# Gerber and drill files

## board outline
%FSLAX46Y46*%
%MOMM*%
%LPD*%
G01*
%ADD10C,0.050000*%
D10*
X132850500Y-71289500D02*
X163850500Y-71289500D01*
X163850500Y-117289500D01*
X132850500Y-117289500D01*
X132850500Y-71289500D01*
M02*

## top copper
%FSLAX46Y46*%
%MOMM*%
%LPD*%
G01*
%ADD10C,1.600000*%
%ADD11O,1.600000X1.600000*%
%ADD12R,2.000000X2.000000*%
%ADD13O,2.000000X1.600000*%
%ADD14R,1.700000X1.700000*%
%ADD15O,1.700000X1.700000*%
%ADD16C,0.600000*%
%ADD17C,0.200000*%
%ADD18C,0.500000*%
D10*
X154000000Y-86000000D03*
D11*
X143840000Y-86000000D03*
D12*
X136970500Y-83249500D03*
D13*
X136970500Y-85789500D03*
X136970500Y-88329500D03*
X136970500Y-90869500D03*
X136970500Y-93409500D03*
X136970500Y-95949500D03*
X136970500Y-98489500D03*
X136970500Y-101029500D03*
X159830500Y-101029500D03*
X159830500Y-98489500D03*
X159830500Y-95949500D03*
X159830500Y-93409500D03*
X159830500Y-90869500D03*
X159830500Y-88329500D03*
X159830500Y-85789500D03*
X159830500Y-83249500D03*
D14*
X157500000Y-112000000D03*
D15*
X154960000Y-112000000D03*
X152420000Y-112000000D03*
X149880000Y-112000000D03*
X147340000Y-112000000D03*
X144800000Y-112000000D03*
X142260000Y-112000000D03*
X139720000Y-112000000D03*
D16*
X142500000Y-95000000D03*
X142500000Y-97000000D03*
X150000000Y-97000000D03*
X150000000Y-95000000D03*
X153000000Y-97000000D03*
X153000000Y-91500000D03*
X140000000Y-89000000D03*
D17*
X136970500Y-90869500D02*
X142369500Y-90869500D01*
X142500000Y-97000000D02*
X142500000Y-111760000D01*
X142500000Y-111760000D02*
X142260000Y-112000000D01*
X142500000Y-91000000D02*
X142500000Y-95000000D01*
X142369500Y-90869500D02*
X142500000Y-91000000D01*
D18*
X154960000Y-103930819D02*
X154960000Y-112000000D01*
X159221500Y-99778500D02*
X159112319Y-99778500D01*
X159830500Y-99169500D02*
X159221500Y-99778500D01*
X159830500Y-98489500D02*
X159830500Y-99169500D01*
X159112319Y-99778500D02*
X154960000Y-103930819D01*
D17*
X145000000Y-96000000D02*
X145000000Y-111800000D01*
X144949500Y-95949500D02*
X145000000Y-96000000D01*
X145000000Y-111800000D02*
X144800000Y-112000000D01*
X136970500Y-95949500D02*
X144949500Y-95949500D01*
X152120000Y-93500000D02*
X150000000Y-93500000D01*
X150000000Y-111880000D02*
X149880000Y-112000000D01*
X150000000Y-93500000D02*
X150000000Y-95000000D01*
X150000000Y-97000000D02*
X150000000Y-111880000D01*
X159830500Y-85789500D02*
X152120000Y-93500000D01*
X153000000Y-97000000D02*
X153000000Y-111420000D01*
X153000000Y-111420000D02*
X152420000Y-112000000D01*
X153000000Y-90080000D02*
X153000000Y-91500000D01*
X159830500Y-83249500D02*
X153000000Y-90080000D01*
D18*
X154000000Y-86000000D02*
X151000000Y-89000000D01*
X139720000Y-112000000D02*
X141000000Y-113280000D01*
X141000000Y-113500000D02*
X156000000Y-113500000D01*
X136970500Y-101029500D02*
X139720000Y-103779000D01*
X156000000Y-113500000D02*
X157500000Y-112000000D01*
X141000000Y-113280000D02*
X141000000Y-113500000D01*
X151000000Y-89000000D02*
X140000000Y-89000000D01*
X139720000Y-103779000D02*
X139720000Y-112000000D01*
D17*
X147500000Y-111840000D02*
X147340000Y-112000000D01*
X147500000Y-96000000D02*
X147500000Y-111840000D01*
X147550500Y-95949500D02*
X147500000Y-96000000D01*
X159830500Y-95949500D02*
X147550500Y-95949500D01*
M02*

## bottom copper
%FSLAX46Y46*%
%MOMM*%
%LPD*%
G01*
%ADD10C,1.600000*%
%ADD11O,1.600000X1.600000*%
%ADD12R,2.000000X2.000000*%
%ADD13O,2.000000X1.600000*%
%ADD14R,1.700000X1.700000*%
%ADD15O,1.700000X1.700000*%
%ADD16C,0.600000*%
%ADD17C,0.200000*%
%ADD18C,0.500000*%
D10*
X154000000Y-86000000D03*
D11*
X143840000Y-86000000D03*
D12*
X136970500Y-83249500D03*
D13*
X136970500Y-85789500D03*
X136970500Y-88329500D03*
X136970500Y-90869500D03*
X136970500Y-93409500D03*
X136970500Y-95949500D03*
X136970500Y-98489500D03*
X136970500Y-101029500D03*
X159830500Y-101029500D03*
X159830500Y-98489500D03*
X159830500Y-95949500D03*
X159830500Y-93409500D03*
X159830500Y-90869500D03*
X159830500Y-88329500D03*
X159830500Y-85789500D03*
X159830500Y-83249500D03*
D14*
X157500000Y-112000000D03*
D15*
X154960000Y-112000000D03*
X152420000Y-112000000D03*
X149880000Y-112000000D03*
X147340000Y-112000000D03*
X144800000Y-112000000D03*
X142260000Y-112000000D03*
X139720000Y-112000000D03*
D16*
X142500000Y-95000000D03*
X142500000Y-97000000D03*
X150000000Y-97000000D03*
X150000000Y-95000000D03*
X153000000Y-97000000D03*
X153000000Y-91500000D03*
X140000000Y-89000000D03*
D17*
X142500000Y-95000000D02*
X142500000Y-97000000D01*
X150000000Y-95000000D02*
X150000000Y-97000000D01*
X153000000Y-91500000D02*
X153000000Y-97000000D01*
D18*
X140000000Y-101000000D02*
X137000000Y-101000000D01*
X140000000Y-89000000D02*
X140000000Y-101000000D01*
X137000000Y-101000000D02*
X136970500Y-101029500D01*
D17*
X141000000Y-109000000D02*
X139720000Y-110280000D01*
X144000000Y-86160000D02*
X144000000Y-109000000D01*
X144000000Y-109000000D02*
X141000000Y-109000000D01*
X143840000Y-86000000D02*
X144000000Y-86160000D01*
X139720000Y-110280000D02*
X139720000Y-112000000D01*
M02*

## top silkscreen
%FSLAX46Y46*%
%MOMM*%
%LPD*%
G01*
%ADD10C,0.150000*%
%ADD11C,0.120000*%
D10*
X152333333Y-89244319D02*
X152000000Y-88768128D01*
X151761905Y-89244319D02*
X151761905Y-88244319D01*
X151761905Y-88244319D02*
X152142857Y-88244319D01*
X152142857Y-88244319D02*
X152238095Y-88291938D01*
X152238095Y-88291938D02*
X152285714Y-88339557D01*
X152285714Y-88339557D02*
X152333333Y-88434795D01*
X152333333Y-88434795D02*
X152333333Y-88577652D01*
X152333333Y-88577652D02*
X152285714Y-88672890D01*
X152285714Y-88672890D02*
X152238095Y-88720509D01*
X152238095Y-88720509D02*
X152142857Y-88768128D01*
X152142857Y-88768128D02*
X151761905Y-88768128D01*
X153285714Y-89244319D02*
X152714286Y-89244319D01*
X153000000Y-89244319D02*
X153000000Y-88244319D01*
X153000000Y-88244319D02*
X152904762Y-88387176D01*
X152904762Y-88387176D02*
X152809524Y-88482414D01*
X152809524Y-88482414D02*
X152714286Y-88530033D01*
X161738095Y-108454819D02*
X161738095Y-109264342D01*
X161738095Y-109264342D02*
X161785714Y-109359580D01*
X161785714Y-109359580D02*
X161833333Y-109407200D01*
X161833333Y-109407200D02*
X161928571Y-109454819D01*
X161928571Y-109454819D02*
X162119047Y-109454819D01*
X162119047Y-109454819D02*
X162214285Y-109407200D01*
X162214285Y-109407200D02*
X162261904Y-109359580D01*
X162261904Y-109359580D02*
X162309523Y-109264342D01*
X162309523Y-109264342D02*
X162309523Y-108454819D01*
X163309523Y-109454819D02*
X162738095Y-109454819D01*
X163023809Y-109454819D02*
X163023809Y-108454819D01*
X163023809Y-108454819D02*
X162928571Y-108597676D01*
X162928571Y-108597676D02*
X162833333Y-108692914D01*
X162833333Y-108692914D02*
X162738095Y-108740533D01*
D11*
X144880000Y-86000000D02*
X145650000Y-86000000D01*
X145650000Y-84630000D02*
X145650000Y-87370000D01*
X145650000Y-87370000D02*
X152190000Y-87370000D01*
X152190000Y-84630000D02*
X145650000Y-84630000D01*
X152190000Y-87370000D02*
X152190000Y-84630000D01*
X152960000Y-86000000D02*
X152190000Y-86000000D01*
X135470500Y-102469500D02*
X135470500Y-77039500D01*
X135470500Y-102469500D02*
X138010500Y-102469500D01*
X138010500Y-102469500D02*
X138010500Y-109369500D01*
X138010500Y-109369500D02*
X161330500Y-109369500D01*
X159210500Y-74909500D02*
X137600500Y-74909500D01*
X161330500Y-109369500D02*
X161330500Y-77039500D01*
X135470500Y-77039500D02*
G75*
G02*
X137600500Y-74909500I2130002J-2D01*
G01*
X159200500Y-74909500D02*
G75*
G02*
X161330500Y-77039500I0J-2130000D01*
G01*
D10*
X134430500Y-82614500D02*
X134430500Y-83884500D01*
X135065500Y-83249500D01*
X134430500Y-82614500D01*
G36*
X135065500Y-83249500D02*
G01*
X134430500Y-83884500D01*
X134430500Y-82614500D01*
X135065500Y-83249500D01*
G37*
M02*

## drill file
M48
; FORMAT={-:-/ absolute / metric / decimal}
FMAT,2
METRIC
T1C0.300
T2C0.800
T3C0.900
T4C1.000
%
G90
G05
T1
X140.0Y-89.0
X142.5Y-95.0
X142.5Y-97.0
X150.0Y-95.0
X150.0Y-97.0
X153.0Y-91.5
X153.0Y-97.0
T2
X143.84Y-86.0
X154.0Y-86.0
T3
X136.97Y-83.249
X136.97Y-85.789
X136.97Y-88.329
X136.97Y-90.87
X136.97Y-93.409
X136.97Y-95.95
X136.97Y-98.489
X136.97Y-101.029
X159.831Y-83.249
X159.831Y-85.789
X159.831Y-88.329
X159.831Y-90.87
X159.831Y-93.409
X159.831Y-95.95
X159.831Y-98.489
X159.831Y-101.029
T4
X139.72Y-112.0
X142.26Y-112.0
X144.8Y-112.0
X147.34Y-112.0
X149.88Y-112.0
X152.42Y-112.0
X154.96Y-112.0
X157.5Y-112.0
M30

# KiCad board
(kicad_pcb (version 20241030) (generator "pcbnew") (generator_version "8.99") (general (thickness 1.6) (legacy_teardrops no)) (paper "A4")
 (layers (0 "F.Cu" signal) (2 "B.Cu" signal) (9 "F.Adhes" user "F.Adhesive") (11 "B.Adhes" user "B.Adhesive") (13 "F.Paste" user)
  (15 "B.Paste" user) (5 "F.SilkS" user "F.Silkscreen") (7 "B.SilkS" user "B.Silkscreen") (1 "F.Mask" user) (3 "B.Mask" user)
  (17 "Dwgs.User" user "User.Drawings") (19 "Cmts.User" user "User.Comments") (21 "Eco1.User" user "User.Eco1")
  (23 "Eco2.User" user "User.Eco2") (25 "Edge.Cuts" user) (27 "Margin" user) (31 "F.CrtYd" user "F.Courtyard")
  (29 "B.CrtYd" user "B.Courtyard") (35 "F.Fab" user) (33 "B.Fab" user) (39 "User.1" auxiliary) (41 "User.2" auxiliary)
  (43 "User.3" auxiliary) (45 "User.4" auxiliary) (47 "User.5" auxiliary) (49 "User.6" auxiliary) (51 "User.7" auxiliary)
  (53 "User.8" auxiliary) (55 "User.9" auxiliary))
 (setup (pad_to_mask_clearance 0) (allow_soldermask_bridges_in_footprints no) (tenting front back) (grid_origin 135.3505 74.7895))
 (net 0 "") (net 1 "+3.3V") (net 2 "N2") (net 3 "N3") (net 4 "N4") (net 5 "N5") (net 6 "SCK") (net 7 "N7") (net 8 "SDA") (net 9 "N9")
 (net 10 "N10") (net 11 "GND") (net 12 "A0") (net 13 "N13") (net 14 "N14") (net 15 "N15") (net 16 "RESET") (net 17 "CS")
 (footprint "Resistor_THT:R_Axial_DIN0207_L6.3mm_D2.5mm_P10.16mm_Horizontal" (layer "F.Cu") (at 154 86 180)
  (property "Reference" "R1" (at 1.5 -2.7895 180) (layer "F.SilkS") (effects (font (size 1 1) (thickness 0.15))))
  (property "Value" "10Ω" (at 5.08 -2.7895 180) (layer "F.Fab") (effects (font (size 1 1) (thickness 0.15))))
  (fp_line (start 9.12 0) (end 8.35 0) (stroke (width 0.12) (type solid)) (layer "F.SilkS"))
  (fp_line (start 8.35 1.37) (end 8.35 -1.37) (stroke (width 0.12) (type solid)) (layer "F.SilkS"))
  (fp_line (start 8.35 -1.37) (end 1.81 -1.37) (stroke (width 0.12) (type solid)) (layer "F.SilkS"))
  (fp_line (start 1.81 1.37) (end 8.35 1.37) (stroke (width 0.12) (type solid)) (layer "F.SilkS"))
  (fp_line (start 1.81 -1.37) (end 1.81 1.37) (stroke (width 0.12) (type solid)) (layer "F.SilkS"))
  (fp_line (start 1.04 0) (end 1.81 0) (stroke (width 0.12) (type solid)) (layer "F.SilkS"))
  (pad "1" thru_hole circle (at 0 0 180) (size 1.6 1.6) (drill 0.8) (layers "F&B.Cu" "*.Mask") (remove_unused_layers no) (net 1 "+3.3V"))
  (pad "2" thru_hole oval (at 10.16 0 180) (size 1.6 1.6) (drill 0.8) (layers "F&B.Cu" "*.Mask") (remove_unused_layers no) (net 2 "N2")))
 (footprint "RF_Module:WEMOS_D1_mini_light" (layer "F.Cu") (at 136.9705 83.2495)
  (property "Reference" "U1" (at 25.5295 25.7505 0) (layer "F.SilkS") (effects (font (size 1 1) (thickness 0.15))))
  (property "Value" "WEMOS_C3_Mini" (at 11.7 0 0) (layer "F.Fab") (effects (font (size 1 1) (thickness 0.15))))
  (fp_line (start -1.5 19.22) (end -1.5 -6.21) (stroke (width 0.12) (type solid)) (layer "F.SilkS"))
  (fp_line (start -1.5 19.22) (end 1.04 19.22) (stroke (width 0.12) (type solid)) (layer "F.SilkS"))
  (fp_line (start 1.04 19.22) (end 1.04 26.12) (stroke (width 0.12) (type solid)) (layer "F.SilkS"))
  (fp_line (start 1.04 26.12) (end 24.36 26.12) (stroke (width 0.12) (type solid)) (layer "F.SilkS"))
  (fp_line (start 22.24 -8.34) (end 0.63 -8.34) (stroke (width 0.12) (type solid)) (layer "F.SilkS"))
  (fp_line (start 24.36 26.12) (end 24.36 -6.21) (stroke (width 0.12) (type solid)) (layer "F.SilkS"))
  (fp_arc (start -1.5 -6.21) (mid -0.876137 -7.716137) (end 0.63 -8.34) (stroke (width 0.12) (type solid)) (layer "F.SilkS"))
  (fp_arc (start 22.23 -8.34) (mid 23.736137 -7.716137) (end 24.36 -6.21) (stroke (width 0.12) (type solid)) (layer "F.SilkS"))
  (fp_poly (pts (xy -2.54 -0.635) (xy -2.54 0.635) (xy -1.905 0)) (stroke (width 0.15) (type solid)) (fill solid) (layer "F.SilkS"))
  (pad "1" thru_hole rect (at 0 0) (size 2 2) (drill 0.9) (layers "*.Cu" "*.Mask") (remove_unused_layers no) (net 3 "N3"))
  (pad "2" thru_hole oval (at 0 2.54) (size 2 1.6) (drill 0.9) (layers "*.Cu" "*.Mask") (remove_unused_layers no) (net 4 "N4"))
  (pad "3" thru_hole oval (at 0 5.08) (size 2 1.6) (drill 0.9) (layers "*.Cu" "*.Mask") (remove_unused_layers no) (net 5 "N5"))
  (pad "4" thru_hole oval (at 0 7.62) (size 2 1.6) (drill 0.9) (layers "*.Cu" "*.Mask") (remove_unused_layers no) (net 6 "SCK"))
  (pad "5" thru_hole oval (at 0 10.16) (size 2 1.6) (drill 0.9) (layers "*.Cu" "*.Mask") (remove_unused_layers no) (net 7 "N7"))
  (pad "6" thru_hole oval (at 0 12.7) (size 2 1.6) (drill 0.9) (layers "*.Cu" "*.Mask") (remove_unused_layers no) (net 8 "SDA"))
  (pad "7" thru_hole oval (at 0 15.24) (size 2 1.6) (drill 0.9) (layers "*.Cu" "*.Mask") (remove_unused_layers no) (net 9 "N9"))
  (pad "8" thru_hole oval (at 0 17.78) (size 2 1.6) (drill 0.9) (layers "*.Cu" "*.Mask") (remove_unused_layers no) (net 1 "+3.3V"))
  (pad "9" thru_hole oval (at 22.86 17.78) (size 2 1.6) (drill 0.9) (layers "*.Cu" "*.Mask") (remove_unused_layers no) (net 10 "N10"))
  (pad "10" thru_hole oval (at 22.86 15.24) (size 2 1.6) (drill 0.9) (layers "*.Cu" "*.Mask") (remove_unused_layers no) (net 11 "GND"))
  (pad "11" thru_hole oval (at 22.86 12.7) (size 2 1.6) (drill 0.9) (layers "*.Cu" "*.Mask") (remove_unused_layers no) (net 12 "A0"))
  (pad "12" thru_hole oval (at 22.86 10.16) (size 2 1.6) (drill 0.9) (layers "*.Cu" "*.Mask") (remove_unused_layers no) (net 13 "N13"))
  (pad "13" thru_hole oval (at 22.86 7.62) (size 2 1.6) (drill 0.9) (layers "*.Cu" "*.Mask") (remove_unused_layers no) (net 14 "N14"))
  (pad "14" thru_hole oval (at 22.86 5.08) (size 2 1.6) (drill 0.9) (layers "*.Cu" "*.Mask") (remove_unused_layers no) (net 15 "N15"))
  (pad "15" thru_hole oval (at 22.86 2.54) (size 2 1.6) (drill 0.9) (layers "*.Cu" "*.Mask") (remove_unused_layers no) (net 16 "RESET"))
  (pad "16" thru_hole oval (at 22.86 0) (size 2 1.6) (drill 0.9) (layers "*.Cu" "*.Mask") (remove_unused_layers no) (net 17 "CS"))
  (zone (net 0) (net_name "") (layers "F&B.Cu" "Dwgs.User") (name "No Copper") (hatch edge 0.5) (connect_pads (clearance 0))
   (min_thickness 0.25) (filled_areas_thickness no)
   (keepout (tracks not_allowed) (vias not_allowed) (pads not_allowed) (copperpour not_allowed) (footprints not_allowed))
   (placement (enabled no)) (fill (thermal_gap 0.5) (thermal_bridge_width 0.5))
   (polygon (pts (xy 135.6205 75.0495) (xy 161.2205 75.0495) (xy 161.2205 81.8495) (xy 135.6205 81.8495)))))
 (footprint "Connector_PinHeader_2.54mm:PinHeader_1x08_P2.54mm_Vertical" (layer "B.Cu") (at 157.5 112 90)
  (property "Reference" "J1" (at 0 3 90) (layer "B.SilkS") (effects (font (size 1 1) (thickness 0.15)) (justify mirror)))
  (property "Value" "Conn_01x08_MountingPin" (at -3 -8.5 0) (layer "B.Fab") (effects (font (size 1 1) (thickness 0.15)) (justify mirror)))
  (pad "1" thru_hole rect (at 0 0 90) (size 1.7 1.7) (drill 1) (layers "F&B.Cu" "*.Mask") (remove_unused_layers no) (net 1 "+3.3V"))
  (pad "2" thru_hole oval (at 0 -2.54 90) (size 1.7 1.7) (drill 1) (layers "F&B.Cu" "*.Mask") (remove_unused_layers no) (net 11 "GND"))
  (pad "3" thru_hole oval (at 0 -5.08 90) (size 1.7 1.7) (drill 1) (layers "F&B.Cu" "*.Mask") (remove_unused_layers no) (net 17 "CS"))
  (pad "4" thru_hole oval (at 0 -7.62 90) (size 1.7 1.7) (drill 1) (layers "F&B.Cu" "*.Mask") (remove_unused_layers no) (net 16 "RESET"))
  (pad "5" thru_hole oval (at 0 -10.16 90) (size 1.7 1.7) (drill 1) (layers "F&B.Cu" "*.Mask") (remove_unused_layers no) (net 12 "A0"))
  (pad "6" thru_hole oval (at 0 -12.7 90) (size 1.7 1.7) (drill 1) (layers "F&B.Cu" "*.Mask") (remove_unused_layers no) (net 8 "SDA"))
  (pad "7" thru_hole oval (at 0 -15.24 90) (size 1.7 1.7) (drill 1) (layers "F&B.Cu" "*.Mask") (remove_unused_layers no) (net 6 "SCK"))
  (pad "8" thru_hole oval (at 0 -17.78 90) (size 1.7 1.7) (drill 1) (layers "F&B.Cu" "*.Mask") (remove_unused_layers no) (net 2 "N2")))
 (gr_rect (start 132.8505 71.2895) (end 163.8505 117.2895) (stroke (width 0.05) (type default)) (fill none) (layer "Edge.Cuts"))
 (segment (start 136.9705 90.8695) (end 142.3695 90.8695) (width 0.2) (layer "F.Cu") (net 6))
 (segment (start 142.5 97) (end 142.5 111.76) (width 0.2) (layer "F.Cu") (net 6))
 (segment (start 142.5 111.76) (end 142.26 112) (width 0.2) (layer "F.Cu") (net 6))
 (segment (start 142.5 91) (end 142.5 95) (width 0.2) (layer "F.Cu") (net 6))
 (segment (start 142.3695 90.8695) (end 142.5 91) (width 0.2) (layer "F.Cu") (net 6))
 (via (at 142.5 95) (size 0.6) (drill 0.3) (layers "F.Cu" "B.Cu") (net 6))
 (via (at 142.5 97) (size 0.6) (drill 0.3) (layers "F.Cu" "B.Cu") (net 6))
 (segment (start 142.5 95) (end 142.5 97) (width 0.2) (layer "B.Cu") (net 6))
 (segment (start 154.96 103.930819) (end 154.96 112) (width 0.5) (layer "F.Cu") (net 11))
 (segment (start 159.2215 99.7785) (end 159.112319 99.7785) (width 0.5) (layer "F.Cu") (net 11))
 (segment (start 159.8305 99.1695) (end 159.2215 99.7785) (width 0.5) (layer "F.Cu") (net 11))
 (segment (start 159.8305 98.4895) (end 159.8305 99.1695) (width 0.5) (layer "F.Cu") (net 11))
 (segment (start 159.112319 99.7785) (end 154.96 103.930819) (width 0.5) (layer "F.Cu") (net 11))
 (segment (start 145 96) (end 145 111.8) (width 0.2) (layer "F.Cu") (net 8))
 (segment (start 144.9495 95.9495) (end 145 96) (width 0.2) (layer "F.Cu") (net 8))
 (segment (start 145 111.8) (end 144.8 112) (width 0.2) (layer "F.Cu") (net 8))
 (segment (start 136.9705 95.9495) (end 144.9495 95.9495) (width 0.2) (layer "F.Cu") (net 8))
 (segment (start 152.12 93.5) (end 150 93.5) (width 0.2) (layer "F.Cu") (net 16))
 (segment (start 150 111.88) (end 149.88 112) (width 0.2) (layer "F.Cu") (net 16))
 (segment (start 150 93.5) (end 150 95) (width 0.2) (layer "F.Cu") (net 16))
 (segment (start 150 97) (end 150 111.88) (width 0.2) (layer "F.Cu") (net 16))
 (segment (start 159.8305 85.7895) (end 152.12 93.5) (width 0.2) (layer "F.Cu") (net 16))
 (via (at 150 97) (size 0.6) (drill 0.3) (layers "F.Cu" "B.Cu") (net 16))
 (via (at 150 95) (size 0.6) (drill 0.3) (layers "F.Cu" "B.Cu") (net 16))
 (segment (start 150 95) (end 150 97) (width 0.2) (layer "B.Cu") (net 16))
 (segment (start 153 97) (end 153 111.42) (width 0.2) (layer "F.Cu") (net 17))
 (segment (start 153 111.42) (end 152.42 112) (width 0.2) (layer "F.Cu") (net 17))
 (segment (start 153 90.08) (end 153 91.5) (width 0.2) (layer "F.Cu") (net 17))
 (segment (start 159.8305 83.2495) (end 153 90.08) (width 0.2) (layer "F.Cu") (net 17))
 (via (at 153 97) (size 0.6) (drill 0.3) (layers "F.Cu" "B.Cu") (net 17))
 (via (at 153 91.5) (size 0.6) (drill 0.3) (layers "F.Cu" "B.Cu") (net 17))
 (segment (start 153 91.5) (end 153 97) (width 0.2) (layer "B.Cu") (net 17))
 (segment (start 154 86) (end 151 89) (width 0.5) (layer "F.Cu") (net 1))
 (segment (start 139.72 112) (end 141 113.28) (width 0.5) (layer "F.Cu") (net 1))
 (segment (start 141 113.5) (end 156 113.5) (width 0.5) (layer "F.Cu") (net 1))
 (segment (start 136.9705 101.0295) (end 139.72 103.779) (width 0.5) (layer "F.Cu") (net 1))
 (segment (start 156 113.5) (end 157.5 112) (width 0.5) (layer "F.Cu") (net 1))
 (segment (start 141 113.28) (end 141 113.5) (width 0.5) (layer "F.Cu") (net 1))
 (segment (start 151 89) (end 140 89) (width 0.5) (layer "F.Cu") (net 1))
 (segment (start 139.72 103.779) (end 139.72 112) (width 0.5) (layer "F.Cu") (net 1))
 (via (at 140 89) (size 0.6) (drill 0.3) (layers "F.Cu" "B.Cu") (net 1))
 (segment (start 140 101) (end 137 101) (width 0.5) (layer "B.Cu") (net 1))
 (segment (start 140 89) (end 140 101) (width 0.5) (layer "B.Cu") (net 1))
 (segment (start 137 101) (end 136.9705 101.0295) (width 0.5) (layer "B.Cu") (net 1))
 (segment (start 147.5 111.84) (end 147.34 112) (width 0.2) (layer "F.Cu") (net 12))
 (segment (start 147.5 96) (end 147.5 111.84) (width 0.2) (layer "F.Cu") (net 12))
 (segment (start 147.5505 95.9495) (end 147.5 96) (width 0.2) (layer "F.Cu") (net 12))
 (segment (start 159.8305 95.9495) (end 147.5505 95.9495) (width 0.2) (layer "F.Cu") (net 12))
 (segment (start 141 109) (end 139.72 110.28) (width 0.2) (layer "B.Cu") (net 2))
 (segment (start 144 86.16) (end 144 109) (width 0.2) (layer "B.Cu") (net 2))
 (segment (start 144 109) (end 141 109) (width 0.2) (layer "B.Cu") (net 2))
 (segment (start 143.84 86) (end 144 86.16) (width 0.2) (layer "B.Cu") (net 2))
 (segment (start 139.72 110.28) (end 139.72 112) (width 0.2) (layer "B.Cu") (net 2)))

